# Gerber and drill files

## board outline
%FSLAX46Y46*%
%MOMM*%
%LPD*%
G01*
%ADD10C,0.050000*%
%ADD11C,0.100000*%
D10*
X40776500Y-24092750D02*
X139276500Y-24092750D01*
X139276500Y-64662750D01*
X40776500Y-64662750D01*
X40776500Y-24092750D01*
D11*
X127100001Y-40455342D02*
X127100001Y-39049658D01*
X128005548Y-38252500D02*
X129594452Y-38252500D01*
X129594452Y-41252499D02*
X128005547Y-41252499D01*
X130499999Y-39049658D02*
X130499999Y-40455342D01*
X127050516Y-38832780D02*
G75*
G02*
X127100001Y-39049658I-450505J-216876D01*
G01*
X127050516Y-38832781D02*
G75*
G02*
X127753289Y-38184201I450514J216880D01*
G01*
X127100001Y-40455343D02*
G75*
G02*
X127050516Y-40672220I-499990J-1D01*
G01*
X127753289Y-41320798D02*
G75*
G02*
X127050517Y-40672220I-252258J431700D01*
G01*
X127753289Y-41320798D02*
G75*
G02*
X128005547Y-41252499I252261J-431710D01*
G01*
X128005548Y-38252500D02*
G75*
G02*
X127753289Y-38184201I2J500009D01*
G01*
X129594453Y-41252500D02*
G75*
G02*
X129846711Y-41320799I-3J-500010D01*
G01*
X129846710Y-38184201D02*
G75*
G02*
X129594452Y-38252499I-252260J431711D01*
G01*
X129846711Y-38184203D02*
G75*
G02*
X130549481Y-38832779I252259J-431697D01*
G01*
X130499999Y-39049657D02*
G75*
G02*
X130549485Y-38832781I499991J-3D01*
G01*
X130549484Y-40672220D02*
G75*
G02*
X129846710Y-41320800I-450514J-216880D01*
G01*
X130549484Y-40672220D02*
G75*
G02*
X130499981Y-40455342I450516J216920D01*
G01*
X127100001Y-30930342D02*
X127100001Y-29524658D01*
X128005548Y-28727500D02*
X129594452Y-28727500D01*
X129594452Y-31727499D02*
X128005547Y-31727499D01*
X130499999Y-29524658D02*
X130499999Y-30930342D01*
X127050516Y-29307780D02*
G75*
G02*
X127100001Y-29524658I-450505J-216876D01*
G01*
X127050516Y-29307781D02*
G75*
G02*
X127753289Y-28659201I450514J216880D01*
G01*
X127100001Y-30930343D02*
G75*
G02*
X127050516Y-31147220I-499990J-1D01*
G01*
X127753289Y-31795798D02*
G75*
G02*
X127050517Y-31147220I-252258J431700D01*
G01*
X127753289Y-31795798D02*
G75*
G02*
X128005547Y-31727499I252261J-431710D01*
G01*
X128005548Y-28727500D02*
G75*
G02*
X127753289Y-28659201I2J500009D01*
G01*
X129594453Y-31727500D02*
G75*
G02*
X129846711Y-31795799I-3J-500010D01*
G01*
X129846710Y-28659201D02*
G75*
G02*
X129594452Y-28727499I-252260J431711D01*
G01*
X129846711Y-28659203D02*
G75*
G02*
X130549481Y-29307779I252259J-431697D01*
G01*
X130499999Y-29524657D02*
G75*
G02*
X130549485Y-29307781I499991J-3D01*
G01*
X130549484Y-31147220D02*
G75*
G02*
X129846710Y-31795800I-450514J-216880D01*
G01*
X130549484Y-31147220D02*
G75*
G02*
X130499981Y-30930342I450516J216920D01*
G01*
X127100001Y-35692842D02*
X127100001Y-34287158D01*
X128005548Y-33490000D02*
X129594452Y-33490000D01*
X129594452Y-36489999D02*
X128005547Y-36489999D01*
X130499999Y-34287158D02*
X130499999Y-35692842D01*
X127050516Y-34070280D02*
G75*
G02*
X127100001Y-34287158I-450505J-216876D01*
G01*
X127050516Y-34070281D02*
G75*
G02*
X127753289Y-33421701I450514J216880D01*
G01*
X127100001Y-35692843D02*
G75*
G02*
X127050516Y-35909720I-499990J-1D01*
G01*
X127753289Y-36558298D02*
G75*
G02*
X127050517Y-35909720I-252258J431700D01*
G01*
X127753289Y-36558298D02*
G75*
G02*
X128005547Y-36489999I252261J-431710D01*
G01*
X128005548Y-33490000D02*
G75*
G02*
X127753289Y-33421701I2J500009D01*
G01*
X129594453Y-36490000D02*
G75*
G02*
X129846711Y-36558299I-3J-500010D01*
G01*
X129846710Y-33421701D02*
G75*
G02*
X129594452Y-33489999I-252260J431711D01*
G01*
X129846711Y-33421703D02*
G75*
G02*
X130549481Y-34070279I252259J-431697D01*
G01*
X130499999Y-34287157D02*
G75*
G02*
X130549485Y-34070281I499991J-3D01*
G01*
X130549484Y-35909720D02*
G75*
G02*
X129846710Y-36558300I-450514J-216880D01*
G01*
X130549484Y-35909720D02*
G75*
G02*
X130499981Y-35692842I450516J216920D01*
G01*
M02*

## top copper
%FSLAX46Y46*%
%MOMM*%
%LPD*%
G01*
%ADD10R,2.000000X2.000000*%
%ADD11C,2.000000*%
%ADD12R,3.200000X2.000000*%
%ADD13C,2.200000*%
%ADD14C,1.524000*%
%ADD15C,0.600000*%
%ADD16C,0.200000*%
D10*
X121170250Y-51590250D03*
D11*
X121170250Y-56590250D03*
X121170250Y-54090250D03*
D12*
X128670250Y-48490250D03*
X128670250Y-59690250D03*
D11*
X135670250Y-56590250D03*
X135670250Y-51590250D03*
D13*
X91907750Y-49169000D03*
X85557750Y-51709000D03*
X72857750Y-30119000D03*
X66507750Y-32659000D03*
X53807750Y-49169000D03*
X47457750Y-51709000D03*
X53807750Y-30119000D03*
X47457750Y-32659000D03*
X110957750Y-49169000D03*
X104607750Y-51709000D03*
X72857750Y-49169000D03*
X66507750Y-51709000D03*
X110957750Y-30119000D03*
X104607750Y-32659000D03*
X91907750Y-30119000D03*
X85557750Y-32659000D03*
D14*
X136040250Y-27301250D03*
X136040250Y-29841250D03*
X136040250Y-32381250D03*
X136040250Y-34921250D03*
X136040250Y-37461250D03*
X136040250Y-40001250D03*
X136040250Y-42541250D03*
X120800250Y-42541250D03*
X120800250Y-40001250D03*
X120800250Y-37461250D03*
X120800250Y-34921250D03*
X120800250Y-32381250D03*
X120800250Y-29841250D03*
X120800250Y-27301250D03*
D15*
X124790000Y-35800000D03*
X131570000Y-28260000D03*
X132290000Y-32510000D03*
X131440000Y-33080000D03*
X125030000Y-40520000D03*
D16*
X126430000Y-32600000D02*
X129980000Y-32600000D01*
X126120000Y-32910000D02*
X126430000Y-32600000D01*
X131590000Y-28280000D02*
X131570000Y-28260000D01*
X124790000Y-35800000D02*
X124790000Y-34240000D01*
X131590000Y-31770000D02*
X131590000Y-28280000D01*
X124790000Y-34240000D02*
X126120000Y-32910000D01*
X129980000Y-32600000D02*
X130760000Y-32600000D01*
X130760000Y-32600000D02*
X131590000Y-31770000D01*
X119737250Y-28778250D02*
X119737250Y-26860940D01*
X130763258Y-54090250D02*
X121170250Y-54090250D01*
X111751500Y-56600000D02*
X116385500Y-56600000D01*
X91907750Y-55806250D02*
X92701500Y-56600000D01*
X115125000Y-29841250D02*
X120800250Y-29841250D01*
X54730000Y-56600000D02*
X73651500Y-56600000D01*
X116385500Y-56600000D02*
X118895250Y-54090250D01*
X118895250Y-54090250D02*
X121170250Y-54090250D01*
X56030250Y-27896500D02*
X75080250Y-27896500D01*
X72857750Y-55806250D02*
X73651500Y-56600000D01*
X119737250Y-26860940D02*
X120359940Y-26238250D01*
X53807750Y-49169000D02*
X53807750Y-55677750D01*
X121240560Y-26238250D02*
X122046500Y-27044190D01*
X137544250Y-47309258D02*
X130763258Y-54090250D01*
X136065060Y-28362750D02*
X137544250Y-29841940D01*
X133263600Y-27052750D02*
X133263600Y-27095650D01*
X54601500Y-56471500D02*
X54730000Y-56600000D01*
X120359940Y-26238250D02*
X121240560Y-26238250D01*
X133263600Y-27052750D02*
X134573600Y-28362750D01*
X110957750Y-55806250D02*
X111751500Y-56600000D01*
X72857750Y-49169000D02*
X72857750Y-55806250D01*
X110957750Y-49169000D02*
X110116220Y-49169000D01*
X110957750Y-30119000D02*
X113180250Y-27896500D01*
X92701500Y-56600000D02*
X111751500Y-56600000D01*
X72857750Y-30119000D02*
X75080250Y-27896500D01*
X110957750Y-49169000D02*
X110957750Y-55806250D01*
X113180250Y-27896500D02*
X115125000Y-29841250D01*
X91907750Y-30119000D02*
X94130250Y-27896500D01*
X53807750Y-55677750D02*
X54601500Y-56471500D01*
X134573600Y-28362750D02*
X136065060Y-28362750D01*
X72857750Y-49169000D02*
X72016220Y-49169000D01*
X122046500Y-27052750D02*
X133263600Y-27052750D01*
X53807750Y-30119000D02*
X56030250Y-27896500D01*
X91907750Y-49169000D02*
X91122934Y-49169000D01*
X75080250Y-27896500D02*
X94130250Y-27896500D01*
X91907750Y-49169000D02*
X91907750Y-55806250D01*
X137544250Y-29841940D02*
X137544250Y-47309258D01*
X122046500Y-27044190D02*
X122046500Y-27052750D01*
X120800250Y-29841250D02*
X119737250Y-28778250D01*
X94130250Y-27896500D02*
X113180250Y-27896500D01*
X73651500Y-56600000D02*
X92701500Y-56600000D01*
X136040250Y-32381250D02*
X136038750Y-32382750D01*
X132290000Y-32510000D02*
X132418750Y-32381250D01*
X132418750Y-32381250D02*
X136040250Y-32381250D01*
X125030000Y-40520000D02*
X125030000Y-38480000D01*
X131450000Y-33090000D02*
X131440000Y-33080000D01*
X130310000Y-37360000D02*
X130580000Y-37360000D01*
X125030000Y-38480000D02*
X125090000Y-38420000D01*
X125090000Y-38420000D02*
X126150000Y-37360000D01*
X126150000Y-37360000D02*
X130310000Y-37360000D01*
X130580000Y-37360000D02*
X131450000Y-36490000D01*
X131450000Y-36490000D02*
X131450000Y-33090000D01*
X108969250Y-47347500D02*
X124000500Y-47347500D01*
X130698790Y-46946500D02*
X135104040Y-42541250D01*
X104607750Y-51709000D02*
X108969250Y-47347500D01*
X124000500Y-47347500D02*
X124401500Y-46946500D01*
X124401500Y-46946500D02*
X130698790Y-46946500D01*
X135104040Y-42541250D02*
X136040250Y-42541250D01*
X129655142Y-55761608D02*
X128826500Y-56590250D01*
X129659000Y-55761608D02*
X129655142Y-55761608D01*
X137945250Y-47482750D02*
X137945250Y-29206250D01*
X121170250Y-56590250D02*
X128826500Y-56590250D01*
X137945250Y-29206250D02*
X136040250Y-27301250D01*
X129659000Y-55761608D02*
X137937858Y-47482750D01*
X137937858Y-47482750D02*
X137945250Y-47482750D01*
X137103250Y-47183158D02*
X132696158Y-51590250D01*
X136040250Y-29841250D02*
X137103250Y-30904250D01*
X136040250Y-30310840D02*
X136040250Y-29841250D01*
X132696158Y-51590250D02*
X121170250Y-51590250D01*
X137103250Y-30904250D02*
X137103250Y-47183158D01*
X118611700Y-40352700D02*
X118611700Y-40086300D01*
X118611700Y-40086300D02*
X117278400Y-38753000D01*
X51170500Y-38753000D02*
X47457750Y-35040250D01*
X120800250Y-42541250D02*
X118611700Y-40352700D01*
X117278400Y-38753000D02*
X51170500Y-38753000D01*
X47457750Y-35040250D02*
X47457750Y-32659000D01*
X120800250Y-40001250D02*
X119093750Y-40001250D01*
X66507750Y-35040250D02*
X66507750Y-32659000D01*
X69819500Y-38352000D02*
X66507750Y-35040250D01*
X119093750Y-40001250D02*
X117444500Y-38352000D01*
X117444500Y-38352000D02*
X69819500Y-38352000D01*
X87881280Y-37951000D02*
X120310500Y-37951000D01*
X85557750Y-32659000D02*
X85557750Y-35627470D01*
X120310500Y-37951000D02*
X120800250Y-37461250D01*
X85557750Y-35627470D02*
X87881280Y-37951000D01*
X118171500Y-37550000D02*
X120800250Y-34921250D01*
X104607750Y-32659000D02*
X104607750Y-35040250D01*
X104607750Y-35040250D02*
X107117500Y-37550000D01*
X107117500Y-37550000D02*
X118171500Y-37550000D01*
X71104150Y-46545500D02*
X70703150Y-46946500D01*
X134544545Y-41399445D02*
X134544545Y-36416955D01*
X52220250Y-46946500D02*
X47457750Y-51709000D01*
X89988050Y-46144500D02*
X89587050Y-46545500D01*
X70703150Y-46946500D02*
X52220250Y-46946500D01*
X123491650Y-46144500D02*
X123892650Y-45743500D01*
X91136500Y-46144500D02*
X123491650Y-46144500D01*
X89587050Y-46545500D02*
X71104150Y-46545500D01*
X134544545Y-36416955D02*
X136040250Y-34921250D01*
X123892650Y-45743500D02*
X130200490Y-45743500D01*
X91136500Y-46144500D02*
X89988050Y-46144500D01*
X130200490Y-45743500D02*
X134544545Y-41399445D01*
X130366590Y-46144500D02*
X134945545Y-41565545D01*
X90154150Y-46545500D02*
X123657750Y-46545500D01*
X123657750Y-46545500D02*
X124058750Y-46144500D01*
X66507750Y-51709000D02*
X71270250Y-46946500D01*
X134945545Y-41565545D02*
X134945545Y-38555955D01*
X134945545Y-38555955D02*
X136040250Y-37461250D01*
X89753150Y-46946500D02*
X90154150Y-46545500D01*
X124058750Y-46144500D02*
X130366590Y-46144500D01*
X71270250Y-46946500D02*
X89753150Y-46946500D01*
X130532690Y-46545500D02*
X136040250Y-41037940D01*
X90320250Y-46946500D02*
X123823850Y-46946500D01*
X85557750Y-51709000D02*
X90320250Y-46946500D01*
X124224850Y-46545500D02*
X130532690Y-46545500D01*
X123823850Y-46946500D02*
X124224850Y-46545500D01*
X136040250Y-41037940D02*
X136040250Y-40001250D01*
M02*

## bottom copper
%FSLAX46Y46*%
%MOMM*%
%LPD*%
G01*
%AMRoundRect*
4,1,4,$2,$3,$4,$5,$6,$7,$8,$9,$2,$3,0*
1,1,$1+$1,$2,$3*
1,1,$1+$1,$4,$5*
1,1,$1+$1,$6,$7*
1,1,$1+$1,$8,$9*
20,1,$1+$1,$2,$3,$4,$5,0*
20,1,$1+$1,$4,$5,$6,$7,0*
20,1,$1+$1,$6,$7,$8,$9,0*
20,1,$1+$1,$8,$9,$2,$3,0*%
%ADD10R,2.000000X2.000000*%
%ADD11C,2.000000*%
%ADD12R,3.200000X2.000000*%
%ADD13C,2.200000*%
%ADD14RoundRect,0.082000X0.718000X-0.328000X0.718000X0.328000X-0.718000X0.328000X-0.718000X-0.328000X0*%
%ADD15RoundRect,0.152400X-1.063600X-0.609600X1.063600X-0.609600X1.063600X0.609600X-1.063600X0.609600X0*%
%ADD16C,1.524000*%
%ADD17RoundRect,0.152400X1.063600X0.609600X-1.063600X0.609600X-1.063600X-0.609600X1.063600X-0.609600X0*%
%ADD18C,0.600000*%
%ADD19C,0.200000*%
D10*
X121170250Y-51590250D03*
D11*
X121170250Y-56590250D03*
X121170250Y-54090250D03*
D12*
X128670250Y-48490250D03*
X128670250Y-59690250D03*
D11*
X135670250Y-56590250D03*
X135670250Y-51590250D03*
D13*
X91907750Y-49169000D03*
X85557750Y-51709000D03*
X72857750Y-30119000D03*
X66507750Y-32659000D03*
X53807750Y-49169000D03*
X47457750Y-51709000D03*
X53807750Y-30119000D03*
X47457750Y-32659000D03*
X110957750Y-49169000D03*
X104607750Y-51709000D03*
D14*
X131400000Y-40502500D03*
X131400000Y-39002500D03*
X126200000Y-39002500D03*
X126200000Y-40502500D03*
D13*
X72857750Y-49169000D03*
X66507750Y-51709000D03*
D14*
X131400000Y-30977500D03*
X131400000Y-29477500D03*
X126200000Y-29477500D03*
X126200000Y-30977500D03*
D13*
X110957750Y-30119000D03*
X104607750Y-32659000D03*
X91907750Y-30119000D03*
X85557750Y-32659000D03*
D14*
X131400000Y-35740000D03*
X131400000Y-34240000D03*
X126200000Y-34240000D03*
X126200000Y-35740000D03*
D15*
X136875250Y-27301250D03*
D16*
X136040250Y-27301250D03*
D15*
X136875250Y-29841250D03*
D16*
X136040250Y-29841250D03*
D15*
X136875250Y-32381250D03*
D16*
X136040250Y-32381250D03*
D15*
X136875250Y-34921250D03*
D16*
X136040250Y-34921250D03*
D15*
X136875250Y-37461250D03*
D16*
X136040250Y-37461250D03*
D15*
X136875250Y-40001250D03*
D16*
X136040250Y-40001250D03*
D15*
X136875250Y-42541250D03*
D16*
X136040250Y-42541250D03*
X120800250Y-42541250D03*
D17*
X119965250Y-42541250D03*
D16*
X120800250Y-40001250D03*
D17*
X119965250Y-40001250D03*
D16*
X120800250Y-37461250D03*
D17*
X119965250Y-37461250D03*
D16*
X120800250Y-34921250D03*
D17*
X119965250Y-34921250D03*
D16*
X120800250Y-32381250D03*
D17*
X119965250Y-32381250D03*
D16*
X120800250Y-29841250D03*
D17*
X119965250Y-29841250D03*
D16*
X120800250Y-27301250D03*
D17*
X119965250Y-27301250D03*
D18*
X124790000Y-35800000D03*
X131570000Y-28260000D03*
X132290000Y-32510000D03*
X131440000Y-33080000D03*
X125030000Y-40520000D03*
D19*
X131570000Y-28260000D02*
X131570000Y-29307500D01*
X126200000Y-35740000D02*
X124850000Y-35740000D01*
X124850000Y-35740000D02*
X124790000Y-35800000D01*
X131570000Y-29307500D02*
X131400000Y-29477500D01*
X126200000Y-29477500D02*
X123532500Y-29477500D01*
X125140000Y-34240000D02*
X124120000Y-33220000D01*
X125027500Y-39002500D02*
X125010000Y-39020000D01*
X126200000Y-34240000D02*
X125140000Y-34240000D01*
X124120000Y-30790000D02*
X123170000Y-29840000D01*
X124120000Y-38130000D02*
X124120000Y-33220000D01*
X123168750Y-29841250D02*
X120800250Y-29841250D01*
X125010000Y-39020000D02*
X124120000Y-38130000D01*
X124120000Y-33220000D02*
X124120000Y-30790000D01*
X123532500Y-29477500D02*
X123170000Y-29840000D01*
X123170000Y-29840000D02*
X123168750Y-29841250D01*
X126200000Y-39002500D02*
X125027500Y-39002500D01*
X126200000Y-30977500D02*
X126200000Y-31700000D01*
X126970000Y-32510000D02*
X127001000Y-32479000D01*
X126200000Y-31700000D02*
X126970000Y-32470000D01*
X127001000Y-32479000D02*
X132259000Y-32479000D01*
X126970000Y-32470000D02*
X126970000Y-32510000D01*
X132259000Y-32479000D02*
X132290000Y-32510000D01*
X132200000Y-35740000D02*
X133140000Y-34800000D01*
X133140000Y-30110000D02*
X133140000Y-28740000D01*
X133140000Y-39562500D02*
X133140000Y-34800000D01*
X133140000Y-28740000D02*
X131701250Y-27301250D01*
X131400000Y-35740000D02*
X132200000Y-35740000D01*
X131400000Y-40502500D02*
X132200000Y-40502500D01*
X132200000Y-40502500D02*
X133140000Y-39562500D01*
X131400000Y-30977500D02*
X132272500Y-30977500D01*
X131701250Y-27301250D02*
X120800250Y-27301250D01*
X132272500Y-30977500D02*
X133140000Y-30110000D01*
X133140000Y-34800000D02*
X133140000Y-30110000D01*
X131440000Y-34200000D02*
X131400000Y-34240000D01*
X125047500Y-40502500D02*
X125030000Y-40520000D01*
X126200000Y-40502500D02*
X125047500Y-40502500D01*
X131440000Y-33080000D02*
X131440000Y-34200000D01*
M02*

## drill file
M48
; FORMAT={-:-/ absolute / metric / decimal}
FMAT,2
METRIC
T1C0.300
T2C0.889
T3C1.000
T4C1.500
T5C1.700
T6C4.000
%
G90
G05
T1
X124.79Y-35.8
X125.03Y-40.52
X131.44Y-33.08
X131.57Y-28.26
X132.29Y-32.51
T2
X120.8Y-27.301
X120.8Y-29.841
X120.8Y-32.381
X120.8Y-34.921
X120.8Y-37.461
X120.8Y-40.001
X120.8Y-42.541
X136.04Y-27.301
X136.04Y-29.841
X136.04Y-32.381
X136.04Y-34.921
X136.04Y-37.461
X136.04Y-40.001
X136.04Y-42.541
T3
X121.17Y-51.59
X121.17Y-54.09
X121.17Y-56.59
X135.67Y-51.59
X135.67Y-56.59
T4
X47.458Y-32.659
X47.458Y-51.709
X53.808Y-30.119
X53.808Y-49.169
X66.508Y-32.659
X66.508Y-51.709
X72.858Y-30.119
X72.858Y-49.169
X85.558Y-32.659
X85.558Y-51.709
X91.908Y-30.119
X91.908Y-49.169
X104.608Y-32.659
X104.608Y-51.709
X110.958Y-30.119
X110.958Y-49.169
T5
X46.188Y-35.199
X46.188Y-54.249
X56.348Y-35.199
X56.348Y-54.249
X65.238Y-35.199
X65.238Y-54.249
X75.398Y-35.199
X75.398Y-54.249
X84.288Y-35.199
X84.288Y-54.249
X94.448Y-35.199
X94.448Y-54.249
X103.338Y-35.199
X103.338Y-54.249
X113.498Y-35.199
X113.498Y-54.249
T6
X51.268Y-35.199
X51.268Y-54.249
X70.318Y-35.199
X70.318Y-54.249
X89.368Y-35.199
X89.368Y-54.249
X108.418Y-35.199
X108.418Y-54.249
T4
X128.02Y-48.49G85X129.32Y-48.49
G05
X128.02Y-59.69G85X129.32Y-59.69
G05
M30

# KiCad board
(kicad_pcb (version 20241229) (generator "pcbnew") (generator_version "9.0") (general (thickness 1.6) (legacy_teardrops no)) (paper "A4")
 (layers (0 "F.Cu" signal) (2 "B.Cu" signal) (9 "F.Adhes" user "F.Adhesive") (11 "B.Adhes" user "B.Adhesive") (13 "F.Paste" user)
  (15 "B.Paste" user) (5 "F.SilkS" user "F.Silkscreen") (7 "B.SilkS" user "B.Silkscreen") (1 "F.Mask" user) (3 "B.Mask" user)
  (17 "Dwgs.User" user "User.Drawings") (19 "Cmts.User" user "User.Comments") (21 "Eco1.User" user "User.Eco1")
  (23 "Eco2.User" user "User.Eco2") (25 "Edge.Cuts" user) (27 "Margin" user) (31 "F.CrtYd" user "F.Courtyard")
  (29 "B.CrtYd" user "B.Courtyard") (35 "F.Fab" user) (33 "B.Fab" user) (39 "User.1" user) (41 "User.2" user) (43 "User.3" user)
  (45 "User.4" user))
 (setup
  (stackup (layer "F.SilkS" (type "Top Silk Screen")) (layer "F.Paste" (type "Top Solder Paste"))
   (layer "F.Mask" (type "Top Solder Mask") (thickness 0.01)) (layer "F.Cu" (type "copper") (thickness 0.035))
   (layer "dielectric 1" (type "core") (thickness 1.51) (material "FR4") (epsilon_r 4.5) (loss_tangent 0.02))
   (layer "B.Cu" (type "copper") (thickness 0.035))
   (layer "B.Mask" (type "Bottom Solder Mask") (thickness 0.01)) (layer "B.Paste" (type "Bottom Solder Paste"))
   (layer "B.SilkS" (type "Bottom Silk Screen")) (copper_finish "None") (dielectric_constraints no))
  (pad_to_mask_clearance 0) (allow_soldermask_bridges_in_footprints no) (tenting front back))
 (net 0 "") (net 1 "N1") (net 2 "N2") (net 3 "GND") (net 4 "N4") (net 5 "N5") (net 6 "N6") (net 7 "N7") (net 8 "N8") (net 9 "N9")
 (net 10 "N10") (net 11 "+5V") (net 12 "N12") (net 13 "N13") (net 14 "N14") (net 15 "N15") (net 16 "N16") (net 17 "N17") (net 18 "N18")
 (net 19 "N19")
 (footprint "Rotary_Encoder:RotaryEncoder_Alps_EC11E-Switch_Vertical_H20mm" (layer "F.Cu") (at 121.17025 51.59025)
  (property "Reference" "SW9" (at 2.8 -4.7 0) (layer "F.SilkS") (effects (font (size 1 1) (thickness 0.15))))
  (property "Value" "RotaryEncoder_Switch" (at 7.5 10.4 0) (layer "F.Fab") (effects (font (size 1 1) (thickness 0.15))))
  (pad "A" thru_hole rect (at 0 0) (size 2 2) (drill 1) (layers "*.Cu" "*.Mask") (remove_unused_layers no) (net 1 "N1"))
  (pad "B" thru_hole circle (at 0 5) (size 2 2) (drill 1) (layers "*.Cu" "*.Mask") (remove_unused_layers no) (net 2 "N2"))
  (pad "C" thru_hole circle (at 0 2.5) (size 2 2) (drill 1) (layers "*.Cu" "*.Mask") (remove_unused_layers no) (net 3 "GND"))
  (pad "MP" thru_hole rect (at 7.5 -3.1) (size 3.2 2) (drill oval 2.8 1.5) (layers "*.Cu" "*.Mask") (remove_unused_layers no))
  (pad "MP" thru_hole rect (at 7.5 8.1) (size 3.2 2) (drill oval 2.8 1.5) (layers "*.Cu" "*.Mask") (remove_unused_layers no))
  (pad "S1" thru_hole circle (at 14.5 5) (size 2 2) (drill 1) (layers "*.Cu" "*.Mask") (remove_unused_layers no) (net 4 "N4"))
  (pad "S2" thru_hole circle (at 14.5 0) (size 2 2) (drill 1) (layers "*.Cu" "*.Mask") (remove_unused_layers no) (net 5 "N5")))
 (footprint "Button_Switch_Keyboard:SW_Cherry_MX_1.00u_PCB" (layer "F.Cu") (at 91.90775 49.169)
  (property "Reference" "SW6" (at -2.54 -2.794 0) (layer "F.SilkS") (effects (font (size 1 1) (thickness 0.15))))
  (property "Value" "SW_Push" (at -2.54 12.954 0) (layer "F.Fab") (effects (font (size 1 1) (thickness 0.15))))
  (pad "" np_thru_hole circle (at -7.62 5.08) (size 1.7 1.7) (drill 1.7) (layers "*.Cu" "*.Mask"))
  (pad "" np_thru_hole circle (at -2.54 5.08) (size 4 4) (drill 4) (layers "*.Cu" "*.Mask"))
  (pad "" np_thru_hole circle (at 2.54 5.08) (size 1.7 1.7) (drill 1.7) (layers "*.Cu" "*.Mask"))
  (pad "1" thru_hole circle (at 0 0) (size 2.2 2.2) (drill 1.5) (layers "*.Cu" "*.Mask") (remove_unused_layers no) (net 3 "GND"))
  (pad "2" thru_hole circle (at -6.35 2.54) (size 2.2 2.2) (drill 1.5) (layers "*.Cu" "*.Mask") (remove_unused_layers no) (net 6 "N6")))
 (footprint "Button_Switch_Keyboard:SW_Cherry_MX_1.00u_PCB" (layer "F.Cu") (at 72.85775 30.119)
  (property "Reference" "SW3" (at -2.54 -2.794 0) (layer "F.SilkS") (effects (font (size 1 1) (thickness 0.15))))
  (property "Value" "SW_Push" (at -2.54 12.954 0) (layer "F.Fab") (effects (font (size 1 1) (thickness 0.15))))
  (pad "" np_thru_hole circle (at -7.62 5.08) (size 1.7 1.7) (drill 1.7) (layers "*.Cu" "*.Mask"))
  (pad "" np_thru_hole circle (at -2.54 5.08) (size 4 4) (drill 4) (layers "*.Cu" "*.Mask"))
  (pad "" np_thru_hole circle (at 2.54 5.08) (size 1.7 1.7) (drill 1.7) (layers "*.Cu" "*.Mask"))
  (pad "1" thru_hole circle (at 0 0) (size 2.2 2.2) (drill 1.5) (layers "*.Cu" "*.Mask") (remove_unused_layers no) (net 3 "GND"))
  (pad "2" thru_hole circle (at -6.35 2.54) (size 2.2 2.2) (drill 1.5) (layers "*.Cu" "*.Mask") (remove_unused_layers no) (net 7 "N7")))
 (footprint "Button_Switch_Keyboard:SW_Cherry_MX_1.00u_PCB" (layer "F.Cu") (at 53.80775 49.169)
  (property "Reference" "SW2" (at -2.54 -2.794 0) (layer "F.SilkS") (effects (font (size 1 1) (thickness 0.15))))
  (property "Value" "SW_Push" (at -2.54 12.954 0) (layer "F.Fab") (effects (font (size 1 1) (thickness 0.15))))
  (pad "" np_thru_hole circle (at -7.62 5.08) (size 1.7 1.7) (drill 1.7) (layers "*.Cu" "*.Mask"))
  (pad "" np_thru_hole circle (at -2.54 5.08) (size 4 4) (drill 4) (layers "*.Cu" "*.Mask"))
  (pad "" np_thru_hole circle (at 2.54 5.08) (size 1.7 1.7) (drill 1.7) (layers "*.Cu" "*.Mask"))
  (pad "1" thru_hole circle (at 0 0) (size 2.2 2.2) (drill 1.5) (layers "*.Cu" "*.Mask") (remove_unused_layers no) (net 3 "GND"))
  (pad "2" thru_hole circle (at -6.35 2.54) (size 2.2 2.2) (drill 1.5) (layers "*.Cu" "*.Mask") (remove_unused_layers no) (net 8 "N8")))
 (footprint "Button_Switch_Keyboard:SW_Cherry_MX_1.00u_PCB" (layer "F.Cu") (at 53.80775 30.119)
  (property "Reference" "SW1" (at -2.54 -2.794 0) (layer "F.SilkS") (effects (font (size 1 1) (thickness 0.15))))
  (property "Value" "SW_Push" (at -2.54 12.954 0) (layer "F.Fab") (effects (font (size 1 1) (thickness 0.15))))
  (pad "" np_thru_hole circle (at -7.62 5.08) (size 1.7 1.7) (drill 1.7) (layers "*.Cu" "*.Mask"))
  (pad "" np_thru_hole circle (at -2.54 5.08) (size 4 4) (drill 4) (layers "*.Cu" "*.Mask"))
  (pad "" np_thru_hole circle (at 2.54 5.08) (size 1.7 1.7) (drill 1.7) (layers "*.Cu" "*.Mask"))
  (pad "1" thru_hole circle (at 0 0) (size 2.2 2.2) (drill 1.5) (layers "*.Cu" "*.Mask") (remove_unused_layers no) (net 3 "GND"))
  (pad "2" thru_hole circle (at -6.35 2.54) (size 2.2 2.2) (drill 1.5) (layers "*.Cu" "*.Mask") (remove_unused_layers no) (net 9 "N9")))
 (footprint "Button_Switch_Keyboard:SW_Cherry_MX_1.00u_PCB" (layer "F.Cu") (at 110.95775 49.169)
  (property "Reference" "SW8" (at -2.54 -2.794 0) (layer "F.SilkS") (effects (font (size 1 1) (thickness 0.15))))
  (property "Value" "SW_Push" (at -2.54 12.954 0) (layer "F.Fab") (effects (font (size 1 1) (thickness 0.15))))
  (pad "" np_thru_hole circle (at -7.62 5.08) (size 1.7 1.7) (drill 1.7) (layers "*.Cu" "*.Mask"))
  (pad "" np_thru_hole circle (at -2.54 5.08) (size 4 4) (drill 4) (layers "*.Cu" "*.Mask"))
  (pad "" np_thru_hole circle (at 2.54 5.08) (size 1.7 1.7) (drill 1.7) (layers "*.Cu" "*.Mask"))
  (pad "1" thru_hole circle (at 0 0) (size 2.2 2.2) (drill 1.5) (layers "*.Cu" "*.Mask") (remove_unused_layers no) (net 3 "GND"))
  (pad "2" thru_hole circle (at -6.35 2.54) (size 2.2 2.2) (drill 1.5) (layers "*.Cu" "*.Mask") (remove_unused_layers no) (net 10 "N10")))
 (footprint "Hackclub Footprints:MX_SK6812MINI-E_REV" (layer "F.Cu") (at 128.8 34.6725)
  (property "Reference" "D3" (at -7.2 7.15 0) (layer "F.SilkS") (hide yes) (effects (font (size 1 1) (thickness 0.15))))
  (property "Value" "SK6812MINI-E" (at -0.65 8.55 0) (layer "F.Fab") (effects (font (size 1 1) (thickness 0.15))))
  (fp_line (start -1.699999 5.782842) (end -1.699999 4.377158) (stroke (width 0.1) (type solid)) (layer "Edge.Cuts"))
  (fp_line (start -0.794452 3.58) (end 0.794452 3.58) (stroke (width 0.1) (type solid)) (layer "Edge.Cuts"))
  (fp_line (start 0.794452 6.579999) (end -0.794453 6.579999) (stroke (width 0.1) (type solid)) (layer "Edge.Cuts"))
  (fp_line (start 1.699999 4.377158) (end 1.699999 5.782842) (stroke (width 0.1) (type solid)) (layer "Edge.Cuts"))
  (fp_arc (start -1.749484 4.16028) (mid -1.712527 4.265932) (end -1.699999 4.377158) (stroke (width 0.1) (type solid)) (layer "Edge.Cuts"))
  (fp_arc (start -1.749484 4.160281) (mid -1.638072 3.575965) (end -1.046711 3.511701) (stroke (width 0.1) (type solid)) (layer "Edge.Cuts"))
  (fp_arc (start -1.699999 5.782843) (mid -1.712527 5.894068) (end -1.749484 5.99972) (stroke (width 0.1) (type solid)) (layer "Edge.Cuts"))
  (fp_arc (start -1.046711 6.648298) (mid -1.638071 6.584034) (end -1.749484 5.99972) (stroke (width 0.1) (type solid)) (layer "Edge.Cuts"))
  (fp_arc (start -1.046711 6.648298) (mid -0.925123 6.597376) (end -0.794453 6.579999) (stroke (width 0.1) (type solid)) (layer "Edge.Cuts"))
  (fp_arc (start -0.794452 3.58) (mid -0.925123 3.562623) (end -1.046711 3.511701) (stroke (width 0.1) (type solid)) (layer "Edge.Cuts"))
  (fp_arc (start 0.794453 6.58) (mid 0.925123 6.597377) (end 1.046711 6.648299) (stroke (width 0.1) (type solid)) (layer "Edge.Cuts"))
  (fp_arc (start 1.04671 3.511701) (mid 0.925122 3.562623) (end 0.794452 3.58) (stroke (width 0.1) (type solid)) (layer "Edge.Cuts"))
  (fp_arc (start 1.046711 3.511703) (mid 1.63807 3.575966) (end 1.749484 4.16028) (stroke (width 0.1) (type solid)) (layer "Edge.Cuts"))
  (fp_arc (start 1.699999 4.377157) (mid 1.712527 4.265932) (end 1.749484 4.16028) (stroke (width 0.1) (type solid)) (layer "Edge.Cuts"))
  (fp_arc (start 1.749484 5.99972) (mid 1.638071 6.584035) (end 1.046711 6.648299) (stroke (width 0.1) (type solid)) (layer "Edge.Cuts"))
  (fp_arc (start 1.749484 5.99972) (mid 1.712527 5.894068) (end 1.699999 5.782842) (stroke (width 0.1) (type solid)) (layer "Edge.Cuts"))
  (pad "1" smd roundrect (at 2.6 5.83 90) (size 0.82 1.6) (layers "B.Cu" "B.Mask" "B.Paste") (roundrect_rratio 0.1) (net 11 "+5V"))
  (pad "2" smd roundrect (at 2.6 4.33 90) (size 0.82 1.6) (layers "B.Cu" "B.Mask" "B.Paste") (roundrect_rratio 0.1) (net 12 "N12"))
  (pad "3" smd roundrect (at -2.6 4.33 90) (size 0.82 1.6) (layers "B.Cu" "B.Mask" "B.Paste") (roundrect_rratio 0.1) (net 3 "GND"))
  (pad "4" smd roundrect (at -2.6 5.83 90) (size 0.82 1.6) (layers "B.Cu" "B.Mask" "B.Paste") (roundrect_rratio 0.1) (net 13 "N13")))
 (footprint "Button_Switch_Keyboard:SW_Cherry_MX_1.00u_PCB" (layer "F.Cu") (at 72.85775 49.169)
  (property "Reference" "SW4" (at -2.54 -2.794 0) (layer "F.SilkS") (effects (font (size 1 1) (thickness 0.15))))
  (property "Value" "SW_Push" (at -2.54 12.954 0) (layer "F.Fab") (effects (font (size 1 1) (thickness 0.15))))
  (pad "" np_thru_hole circle (at -7.62 5.08) (size 1.7 1.7) (drill 1.7) (layers "*.Cu" "*.Mask"))
  (pad "" np_thru_hole circle (at -2.54 5.08) (size 4 4) (drill 4) (layers "*.Cu" "*.Mask"))
  (pad "" np_thru_hole circle (at 2.54 5.08) (size 1.7 1.7) (drill 1.7) (layers "*.Cu" "*.Mask"))
  (pad "1" thru_hole circle (at 0 0) (size 2.2 2.2) (drill 1.5) (layers "*.Cu" "*.Mask") (remove_unused_layers no) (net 3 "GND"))
  (pad "2" thru_hole circle (at -6.35 2.54) (size 2.2 2.2) (drill 1.5) (layers "*.Cu" "*.Mask") (remove_unused_layers no) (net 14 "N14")))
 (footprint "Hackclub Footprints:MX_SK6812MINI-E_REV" (layer "F.Cu") (at 128.8 25.1475)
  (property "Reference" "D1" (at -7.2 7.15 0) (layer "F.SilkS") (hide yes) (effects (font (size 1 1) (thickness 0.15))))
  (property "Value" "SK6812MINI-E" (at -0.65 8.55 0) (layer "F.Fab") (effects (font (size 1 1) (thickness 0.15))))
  (fp_line (start -1.699999 5.782842) (end -1.699999 4.377158) (stroke (width 0.1) (type solid)) (layer "Edge.Cuts"))
  (fp_line (start -0.794452 3.58) (end 0.794452 3.58) (stroke (width 0.1) (type solid)) (layer "Edge.Cuts"))
  (fp_line (start 0.794452 6.579999) (end -0.794453 6.579999) (stroke (width 0.1) (type solid)) (layer "Edge.Cuts"))
  (fp_line (start 1.699999 4.377158) (end 1.699999 5.782842) (stroke (width 0.1) (type solid)) (layer "Edge.Cuts"))
  (fp_arc (start -1.749484 4.16028) (mid -1.712527 4.265932) (end -1.699999 4.377158) (stroke (width 0.1) (type solid)) (layer "Edge.Cuts"))
  (fp_arc (start -1.749484 4.160281) (mid -1.638072 3.575965) (end -1.046711 3.511701) (stroke (width 0.1) (type solid)) (layer "Edge.Cuts"))
  (fp_arc (start -1.699999 5.782843) (mid -1.712527 5.894068) (end -1.749484 5.99972) (stroke (width 0.1) (type solid)) (layer "Edge.Cuts"))
  (fp_arc (start -1.046711 6.648298) (mid -1.638071 6.584034) (end -1.749484 5.99972) (stroke (width 0.1) (type solid)) (layer "Edge.Cuts"))
  (fp_arc (start -1.046711 6.648298) (mid -0.925123 6.597376) (end -0.794453 6.579999) (stroke (width 0.1) (type solid)) (layer "Edge.Cuts"))
  (fp_arc (start -0.794452 3.58) (mid -0.925123 3.562623) (end -1.046711 3.511701) (stroke (width 0.1) (type solid)) (layer "Edge.Cuts"))
  (fp_arc (start 0.794453 6.58) (mid 0.925123 6.597377) (end 1.046711 6.648299) (stroke (width 0.1) (type solid)) (layer "Edge.Cuts"))
  (fp_arc (start 1.04671 3.511701) (mid 0.925122 3.562623) (end 0.794452 3.58) (stroke (width 0.1) (type solid)) (layer "Edge.Cuts"))
  (fp_arc (start 1.046711 3.511703) (mid 1.63807 3.575966) (end 1.749484 4.16028) (stroke (width 0.1) (type solid)) (layer "Edge.Cuts"))
  (fp_arc (start 1.699999 4.377157) (mid 1.712527 4.265932) (end 1.749484 4.16028) (stroke (width 0.1) (type solid)) (layer "Edge.Cuts"))
  (fp_arc (start 1.749484 5.99972) (mid 1.638071 6.584035) (end 1.046711 6.648299) (stroke (width 0.1) (type solid)) (layer "Edge.Cuts"))
  (fp_arc (start 1.749484 5.99972) (mid 1.712527 5.894068) (end 1.699999 5.782842) (stroke (width 0.1) (type solid)) (layer "Edge.Cuts"))
  (pad "1" smd roundrect (at 2.6 5.83 90) (size 0.82 1.6) (layers "B.Cu" "B.Mask" "B.Paste") (roundrect_rratio 0.1) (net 11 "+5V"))
  (pad "2" smd roundrect (at 2.6 4.33 90) (size 0.82 1.6) (layers "B.Cu" "B.Mask" "B.Paste") (roundrect_rratio 0.1) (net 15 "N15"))
  (pad "3" smd roundrect (at -2.6 4.33 90) (size 0.82 1.6) (layers "B.Cu" "B.Mask" "B.Paste") (roundrect_rratio 0.1) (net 3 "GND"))
  (pad "4" smd roundrect (at -2.6 5.83 90) (size 0.82 1.6) (layers "B.Cu" "B.Mask" "B.Paste") (roundrect_rratio 0.1) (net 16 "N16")))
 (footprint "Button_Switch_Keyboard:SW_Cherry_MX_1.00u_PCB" (layer "F.Cu") (at 110.95775 30.119)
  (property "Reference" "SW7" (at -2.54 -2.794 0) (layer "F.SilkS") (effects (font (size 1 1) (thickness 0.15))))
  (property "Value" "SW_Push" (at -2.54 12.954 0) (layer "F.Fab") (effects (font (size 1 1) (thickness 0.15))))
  (pad "" np_thru_hole circle (at -7.62 5.08) (size 1.7 1.7) (drill 1.7) (layers "*.Cu" "*.Mask"))
  (pad "" np_thru_hole circle (at -2.54 5.08) (size 4 4) (drill 4) (layers "*.Cu" "*.Mask"))
  (pad "" np_thru_hole circle (at 2.54 5.08) (size 1.7 1.7) (drill 1.7) (layers "*.Cu" "*.Mask"))
  (pad "1" thru_hole circle (at 0 0) (size 2.2 2.2) (drill 1.5) (layers "*.Cu" "*.Mask") (remove_unused_layers no) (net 3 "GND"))
  (pad "2" thru_hole circle (at -6.35 2.54) (size 2.2 2.2) (drill 1.5) (layers "*.Cu" "*.Mask") (remove_unused_layers no) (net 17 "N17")))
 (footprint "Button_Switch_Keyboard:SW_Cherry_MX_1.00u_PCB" (layer "F.Cu") (at 91.90775 30.119)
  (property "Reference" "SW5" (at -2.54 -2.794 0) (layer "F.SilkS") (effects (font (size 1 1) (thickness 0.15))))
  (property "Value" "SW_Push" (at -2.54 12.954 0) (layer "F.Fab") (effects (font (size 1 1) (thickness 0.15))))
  (pad "" np_thru_hole circle (at -7.62 5.08) (size 1.7 1.7) (drill 1.7) (layers "*.Cu" "*.Mask"))
  (pad "" np_thru_hole circle (at -2.54 5.08) (size 4 4) (drill 4) (layers "*.Cu" "*.Mask"))
  (pad "" np_thru_hole circle (at 2.54 5.08) (size 1.7 1.7) (drill 1.7) (layers "*.Cu" "*.Mask"))
  (pad "1" thru_hole circle (at 0 0) (size 2.2 2.2) (drill 1.5) (layers "*.Cu" "*.Mask") (remove_unused_layers no) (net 3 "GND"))
  (pad "2" thru_hole circle (at -6.35 2.54) (size 2.2 2.2) (drill 1.5) (layers "*.Cu" "*.Mask") (remove_unused_layers no) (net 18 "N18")))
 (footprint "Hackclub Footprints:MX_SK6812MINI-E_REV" (layer "F.Cu") (at 128.8 29.91)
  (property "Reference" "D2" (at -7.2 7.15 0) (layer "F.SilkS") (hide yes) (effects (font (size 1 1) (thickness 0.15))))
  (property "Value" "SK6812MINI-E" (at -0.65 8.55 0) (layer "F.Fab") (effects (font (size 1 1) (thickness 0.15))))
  (fp_line (start -1.699999 5.782842) (end -1.699999 4.377158) (stroke (width 0.1) (type solid)) (layer "Edge.Cuts"))
  (fp_line (start -0.794452 3.58) (end 0.794452 3.58) (stroke (width 0.1) (type solid)) (layer "Edge.Cuts"))
  (fp_line (start 0.794452 6.579999) (end -0.794453 6.579999) (stroke (width 0.1) (type solid)) (layer "Edge.Cuts"))
  (fp_line (start 1.699999 4.377158) (end 1.699999 5.782842) (stroke (width 0.1) (type solid)) (layer "Edge.Cuts"))
  (fp_arc (start -1.749484 4.16028) (mid -1.712527 4.265932) (end -1.699999 4.377158) (stroke (width 0.1) (type solid)) (layer "Edge.Cuts"))
  (fp_arc (start -1.749484 4.160281) (mid -1.638072 3.575965) (end -1.046711 3.511701) (stroke (width 0.1) (type solid)) (layer "Edge.Cuts"))
  (fp_arc (start -1.699999 5.782843) (mid -1.712527 5.894068) (end -1.749484 5.99972) (stroke (width 0.1) (type solid)) (layer "Edge.Cuts"))
  (fp_arc (start -1.046711 6.648298) (mid -1.638071 6.584034) (end -1.749484 5.99972) (stroke (width 0.1) (type solid)) (layer "Edge.Cuts"))
  (fp_arc (start -1.046711 6.648298) (mid -0.925123 6.597376) (end -0.794453 6.579999) (stroke (width 0.1) (type solid)) (layer "Edge.Cuts"))
  (fp_arc (start -0.794452 3.58) (mid -0.925123 3.562623) (end -1.046711 3.511701) (stroke (width 0.1) (type solid)) (layer "Edge.Cuts"))
  (fp_arc (start 0.794453 6.58) (mid 0.925123 6.597377) (end 1.046711 6.648299) (stroke (width 0.1) (type solid)) (layer "Edge.Cuts"))
  (fp_arc (start 1.04671 3.511701) (mid 0.925122 3.562623) (end 0.794452 3.58) (stroke (width 0.1) (type solid)) (layer "Edge.Cuts"))
  (fp_arc (start 1.046711 3.511703) (mid 1.63807 3.575966) (end 1.749484 4.16028) (stroke (width 0.1) (type solid)) (layer "Edge.Cuts"))
  (fp_arc (start 1.699999 4.377157) (mid 1.712527 4.265932) (end 1.749484 4.16028) (stroke (width 0.1) (type solid)) (layer "Edge.Cuts"))
  (fp_arc (start 1.749484 5.99972) (mid 1.638071 6.584035) (end 1.046711 6.648299) (stroke (width 0.1) (type solid)) (layer "Edge.Cuts"))
  (fp_arc (start 1.749484 5.99972) (mid 1.712527 5.894068) (end 1.699999 5.782842) (stroke (width 0.1) (type solid)) (layer "Edge.Cuts"))
  (pad "1" smd roundrect (at 2.6 5.83 90) (size 0.82 1.6) (layers "B.Cu" "B.Mask" "B.Paste") (roundrect_rratio 0.1) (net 11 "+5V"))
  (pad "2" smd roundrect (at 2.6 4.33 90) (size 0.82 1.6) (layers "B.Cu" "B.Mask" "B.Paste") (roundrect_rratio 0.1) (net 13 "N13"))
  (pad "3" smd roundrect (at -2.6 4.33 90) (size 0.82 1.6) (layers "B.Cu" "B.Mask" "B.Paste") (roundrect_rratio 0.1) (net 3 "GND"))
  (pad "4" smd roundrect (at -2.6 5.83 90) (size 0.82 1.6) (layers "B.Cu" "B.Mask" "B.Paste") (roundrect_rratio 0.1) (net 15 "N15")))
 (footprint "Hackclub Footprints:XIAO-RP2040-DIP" (layer "B.Cu") (at 128.42025 34.92125 180)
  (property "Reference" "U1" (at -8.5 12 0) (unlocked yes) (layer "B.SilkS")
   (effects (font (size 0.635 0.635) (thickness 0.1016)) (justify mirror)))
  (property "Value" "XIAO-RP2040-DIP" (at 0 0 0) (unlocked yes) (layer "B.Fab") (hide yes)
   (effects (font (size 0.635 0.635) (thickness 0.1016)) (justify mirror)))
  (pad "1" smd roundrect (at -8.455 7.62) (size 2.432 1.524) (layers "B.Cu" "B.Mask") (roundrect_rratio 0.1) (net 2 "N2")
   (thermal_bridge_angle 45))
  (pad "1" thru_hole circle (at -7.62 7.62) (size 1.524 1.524) (drill 0.889) (layers "*.Cu" "*.Mask") (remove_unused_layers no) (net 2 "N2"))
  (pad "2" smd roundrect (at -8.455 5.08) (size 2.432 1.524) (layers "B.Cu" "B.Mask") (roundrect_rratio 0.1) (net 1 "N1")
   (thermal_bridge_angle 45))
  (pad "2" thru_hole circle (at -7.62 5.08) (size 1.524 1.524) (drill 0.889) (layers "*.Cu" "*.Mask") (remove_unused_layers no) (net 1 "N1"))
  (pad "3" smd roundrect (at -8.455 2.54) (size 2.432 1.524) (layers "B.Cu" "B.Mask") (roundrect_rratio 0.1) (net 16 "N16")
   (thermal_bridge_angle 45))
  (pad "3" thru_hole circle (at -7.62 2.54) (size 1.524 1.524) (drill 0.889) (layers "*.Cu" "*.Mask") (remove_unused_layers no)
   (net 16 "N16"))
  (pad "4" smd roundrect (at -8.455 0) (size 2.432 1.524) (layers "B.Cu" "B.Mask") (roundrect_rratio 0.1) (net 8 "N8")
   (thermal_bridge_angle 45))
  (pad "4" thru_hole circle (at -7.62 0) (size 1.524 1.524) (drill 0.889) (layers "*.Cu" "*.Mask") (remove_unused_layers no) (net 8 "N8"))
  (pad "5" smd roundrect (at -8.455 -2.54) (size 2.432 1.524) (layers "B.Cu" "B.Mask") (roundrect_rratio 0.1) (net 14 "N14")
   (thermal_bridge_angle 45))
  (pad "5" thru_hole circle (at -7.62 -2.54) (size 1.524 1.524) (drill 0.889) (layers "*.Cu" "*.Mask") (remove_unused_layers no)
   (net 14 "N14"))
  (pad "6" smd roundrect (at -8.455 -5.08) (size 2.432 1.524) (layers "B.Cu" "B.Mask") (roundrect_rratio 0.1) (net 6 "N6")
   (thermal_bridge_angle 45))
  (pad "6" thru_hole circle (at -7.62 -5.08) (size 1.524 1.524) (drill 0.889) (layers "*.Cu" "*.Mask") (remove_unused_layers no)
   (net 6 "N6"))
  (pad "7" smd roundrect (at -8.455 -7.62) (size 2.432 1.524) (layers "B.Cu" "B.Mask") (roundrect_rratio 0.1) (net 10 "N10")
   (thermal_bridge_angle 45))
  (pad "7" thru_hole circle (at -7.62 -7.62) (size 1.524 1.524) (drill 0.889) (layers "*.Cu" "*.Mask") (remove_unused_layers no)
   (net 10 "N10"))
  (pad "8" thru_hole circle (at 7.62 -7.62 180) (size 1.524 1.524) (drill 0.889) (layers "*.Cu" "*.Mask") (remove_unused_layers no)
   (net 9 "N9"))
  (pad "8" smd roundrect (at 8.455 -7.62 180) (size 2.432 1.524) (layers "B.Cu" "B.Mask") (roundrect_rratio 0.1) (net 9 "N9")
   (thermal_bridge_angle 45))
  (pad "9" thru_hole circle (at 7.62 -5.08 180) (size 1.524 1.524) (drill 0.889) (layers "*.Cu" "*.Mask") (remove_unused_layers no)
   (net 7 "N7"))
  (pad "9" smd roundrect (at 8.455 -5.08 180) (size 2.432 1.524) (layers "B.Cu" "B.Mask") (roundrect_rratio 0.1) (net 7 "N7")
   (thermal_bridge_angle 45))
  (pad "10" thru_hole circle (at 7.62 -2.54 180) (size 1.524 1.524) (drill 0.889) (layers "*.Cu" "*.Mask") (remove_unused_layers no)
   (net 18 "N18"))
  (pad "10" smd roundrect (at 8.455 -2.54 180) (size 2.432 1.524) (layers "B.Cu" "B.Mask") (roundrect_rratio 0.1) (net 18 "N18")
   (thermal_bridge_angle 45))
  (pad "11" thru_hole circle (at 7.62 0 180) (size 1.524 1.524) (drill 0.889) (layers "*.Cu" "*.Mask") (remove_unused_layers no)
   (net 17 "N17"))
  (pad "11" smd roundrect (at 8.455 0 180) (size 2.432 1.524) (layers "B.Cu" "B.Mask") (roundrect_rratio 0.1) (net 17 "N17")
   (thermal_bridge_angle 45))
  (pad "12" thru_hole circle (at 7.62 2.54 180) (size 1.524 1.524) (drill 0.889) (layers "*.Cu" "*.Mask") (remove_unused_layers no)
   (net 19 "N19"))
  (pad "12" smd roundrect (at 8.455 2.54 180) (size 2.432 1.524) (layers "B.Cu" "B.Mask") (roundrect_rratio 0.1) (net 19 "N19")
   (thermal_bridge_angle 45))
  (pad "13" thru_hole circle (at 7.62 5.08 180) (size 1.524 1.524) (drill 0.889) (layers "*.Cu" "*.Mask") (remove_unused_layers no)
   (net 3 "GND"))
  (pad "13" smd roundrect (at 8.455 5.08 180) (size 2.432 1.524) (layers "B.Cu" "B.Mask") (roundrect_rratio 0.1) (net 3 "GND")
   (thermal_bridge_angle 45))
  (pad "14" thru_hole circle (at 7.62 7.62 180) (size 1.524 1.524) (drill 0.889) (layers "*.Cu" "*.Mask") (remove_unused_layers no)
   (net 11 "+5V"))
  (pad "14" smd roundrect (at 8.455 7.62 180) (size 2.432 1.524) (layers "B.Cu" "B.Mask") (roundrect_rratio 0.1) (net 11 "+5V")
   (thermal_bridge_angle 45)))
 (gr_rect (start 40.7765 24.09275) (end 139.2765 64.66275) (stroke (width 0.05) (type default)) (fill no) (layer "Edge.Cuts"))
 (segment (start 126.43 32.6) (end 129.98 32.6) (width 0.2) (layer "F.Cu") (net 15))
 (segment (start 126.12 32.91) (end 126.43 32.6) (width 0.2) (layer "F.Cu") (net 15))
 (segment (start 131.59 28.28) (end 131.57 28.26) (width 0.2) (layer "F.Cu") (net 15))
 (segment (start 124.79 35.8) (end 124.79 34.24) (width 0.2) (layer "F.Cu") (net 15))
 (segment (start 131.59 31.77) (end 131.59 28.28) (width 0.2) (layer "F.Cu") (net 15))
 (segment (start 124.79 34.24) (end 126.12 32.91) (width 0.2) (layer "F.Cu") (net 15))
 (segment (start 129.98 32.6) (end 130.76 32.6) (width 0.2) (layer "F.Cu") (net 15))
 (segment (start 130.76 32.6) (end 131.59 31.77) (width 0.2) (layer "F.Cu") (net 15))
 (via (at 124.79 35.8) (size 0.6) (drill 0.3) (layers "F.Cu" "B.Cu") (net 15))
 (via (at 131.57 28.26) (size 0.6) (drill 0.3) (layers "F.Cu" "B.Cu") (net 15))
 (segment (start 131.57 28.26) (end 131.57 29.3075) (width 0.2) (layer "B.Cu") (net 15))
 (segment (start 126.2 35.74) (end 124.85 35.74) (width 0.2) (layer "B.Cu") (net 15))
 (segment (start 124.85 35.74) (end 124.79 35.8) (width 0.2) (layer "B.Cu") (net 15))
 (segment (start 131.57 29.3075) (end 131.4 29.4775) (width 0.2) (layer "B.Cu") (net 15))
 (segment (start 119.73725 28.77825) (end 119.73725 26.86094) (width 0.2) (layer "F.Cu") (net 3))
 (segment (start 130.763258 54.09025) (end 121.17025 54.09025) (width 0.2) (layer "F.Cu") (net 3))
 (segment (start 111.7515 56.6) (end 116.3855 56.6) (width 0.2) (layer "F.Cu") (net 3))
 (segment (start 91.90775 55.80625) (end 92.7015 56.6) (width 0.2) (layer "F.Cu") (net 3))
 (segment (start 115.125 29.84125) (end 120.80025 29.84125) (width 0.2) (layer "F.Cu") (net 3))
 (segment (start 54.73 56.6) (end 73.6515 56.6) (width 0.2) (layer "F.Cu") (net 3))
 (segment (start 116.3855 56.6) (end 118.89525 54.09025) (width 0.2) (layer "F.Cu") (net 3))
 (segment (start 118.89525 54.09025) (end 121.17025 54.09025) (width 0.2) (layer "F.Cu") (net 3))
 (segment (start 56.03025 27.8965) (end 75.08025 27.8965) (width 0.2) (layer "F.Cu") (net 3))
 (segment (start 72.85775 55.80625) (end 73.6515 56.6) (width 0.2) (layer "F.Cu") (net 3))
 (segment (start 119.73725 26.86094) (end 120.35994 26.23825) (width 0.2) (layer "F.Cu") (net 3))
 (segment (start 53.80775 49.169) (end 53.80775 55.67775) (width 0.2) (layer "F.Cu") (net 3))
 (segment (start 121.24056 26.23825) (end 122.0465 27.04419) (width 0.2) (layer "F.Cu") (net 3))
 (segment (start 137.54425 47.309258) (end 130.763258 54.09025) (width 0.2) (layer "F.Cu") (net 3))
 (segment (start 136.06506 28.36275) (end 137.54425 29.84194) (width 0.2) (layer "F.Cu") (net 3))
 (segment (start 133.2636 27.05275) (end 133.2636 27.09565) (width 0.2) (layer "F.Cu") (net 3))
 (segment (start 54.6015 56.4715) (end 54.73 56.6) (width 0.2) (layer "F.Cu") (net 3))
 (segment (start 120.35994 26.23825) (end 121.24056 26.23825) (width 0.2) (layer "F.Cu") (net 3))
 (segment (start 133.2636 27.05275) (end 134.5736 28.36275) (width 0.2) (layer "F.Cu") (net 3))
 (segment (start 110.95775 55.80625) (end 111.7515 56.6) (width 0.2) (layer "F.Cu") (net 3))
 (segment (start 72.85775 49.169) (end 72.85775 55.80625) (width 0.2) (layer "F.Cu") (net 3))
 (segment (start 110.95775 49.169) (end 110.11622 49.169) (width 0.2) (layer "F.Cu") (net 3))
 (segment (start 110.95775 30.119) (end 113.18025 27.8965) (width 0.2) (layer "F.Cu") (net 3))
 (segment (start 92.7015 56.6) (end 111.7515 56.6) (width 0.2) (layer "F.Cu") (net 3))
 (segment (start 72.85775 30.119) (end 75.08025 27.8965) (width 0.2) (layer "F.Cu") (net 3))
 (segment (start 110.95775 49.169) (end 110.95775 55.80625) (width 0.2) (layer "F.Cu") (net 3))
 (segment (start 113.18025 27.8965) (end 115.125 29.84125) (width 0.2) (layer "F.Cu") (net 3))
 (segment (start 91.90775 30.119) (end 94.13025 27.8965) (width 0.2) (layer "F.Cu") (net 3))
 (segment (start 53.80775 55.67775) (end 54.6015 56.4715) (width 0.2) (layer "F.Cu") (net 3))
 (segment (start 134.5736 28.36275) (end 136.06506 28.36275) (width 0.2) (layer "F.Cu") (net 3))
 (segment (start 72.85775 49.169) (end 72.01622 49.169) (width 0.2) (layer "F.Cu") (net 3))
 (segment (start 122.0465 27.05275) (end 133.2636 27.05275) (width 0.2) (layer "F.Cu") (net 3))
 (segment (start 53.80775 30.119) (end 56.03025 27.8965) (width 0.2) (layer "F.Cu") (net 3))
 (segment (start 91.90775 49.169) (end 91.122934 49.169) (width 0.2) (layer "F.Cu") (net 3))
 (segment (start 75.08025 27.8965) (end 94.13025 27.8965) (width 0.2) (layer "F.Cu") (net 3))
 (segment (start 91.90775 49.169) (end 91.90775 55.80625) (width 0.2) (layer "F.Cu") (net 3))
 (segment (start 137.54425 29.84194) (end 137.54425 47.309258) (width 0.2) (layer "F.Cu") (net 3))
 (segment (start 122.0465 27.04419) (end 122.0465 27.05275) (width 0.2) (layer "F.Cu") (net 3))
 (segment (start 120.80025 29.84125) (end 119.73725 28.77825) (width 0.2) (layer "F.Cu") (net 3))
 (segment (start 94.13025 27.8965) (end 113.18025 27.8965) (width 0.2) (layer "F.Cu") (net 3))
 (segment (start 73.6515 56.6) (end 92.7015 56.6) (width 0.2) (layer "F.Cu") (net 3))
 (segment (start 126.2 29.4775) (end 123.5325 29.4775) (width 0.2) (layer "B.Cu") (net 3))
 (segment (start 125.14 34.24) (end 124.12 33.22) (width 0.2) (layer "B.Cu") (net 3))
 (segment (start 125.0275 39.0025) (end 125.01 39.02) (width 0.2) (layer "B.Cu") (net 3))
 (segment (start 126.2 34.24) (end 125.14 34.24) (width 0.2) (layer "B.Cu") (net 3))
 (segment (start 124.12 30.79) (end 123.17 29.84) (width 0.2) (layer "B.Cu") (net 3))
 (segment (start 124.12 38.13) (end 124.12 33.22) (width 0.2) (layer "B.Cu") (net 3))
 (segment (start 123.16875 29.84125) (end 120.80025 29.84125) (width 0.2) (layer "B.Cu") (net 3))
 (segment (start 125.01 39.02) (end 124.12 38.13) (width 0.2) (layer "B.Cu") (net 3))
 (segment (start 124.12 33.22) (end 124.12 30.79) (width 0.2) (layer "B.Cu") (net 3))
 (segment (start 123.5325 29.4775) (end 123.17 29.84) (width 0.2) (layer "B.Cu") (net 3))
 (segment (start 123.17 29.84) (end 123.16875 29.84125) (width 0.2) (layer "B.Cu") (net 3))
 (segment (start 126.2 39.0025) (end 125.0275 39.0025) (width 0.2) (layer "B.Cu") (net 3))
 (segment (start 136.04025 32.38125) (end 136.03875 32.38275) (width 0.2) (layer "F.Cu") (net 16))
 (segment (start 132.29 32.51) (end 132.41875 32.38125) (width 0.2) (layer "F.Cu") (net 16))
 (segment (start 132.41875 32.38125) (end 136.04025 32.38125) (width 0.2) (layer "F.Cu") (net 16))
 (via (at 132.29 32.51) (size 0.6) (drill 0.3) (layers "F.Cu" "B.Cu") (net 16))
 (segment (start 126.2 30.9775) (end 126.2 31.7) (width 0.2) (layer "B.Cu") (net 16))
 (segment (start 126.97 32.51) (end 127.001 32.479) (width 0.2) (layer "B.Cu") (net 16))
 (segment (start 126.2 31.7) (end 126.97 32.47) (width 0.2) (layer "B.Cu") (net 16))
 (segment (start 127.001 32.479) (end 132.259 32.479) (width 0.2) (layer "B.Cu") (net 16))
 (segment (start 126.97 32.47) (end 126.97 32.51) (width 0.2) (layer "B.Cu") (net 16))
 (segment (start 132.259 32.479) (end 132.29 32.51) (width 0.2) (layer "B.Cu") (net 16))
 (segment (start 132.2 35.74) (end 133.14 34.8) (width 0.2) (layer "B.Cu") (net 11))
 (segment (start 133.14 30.11) (end 133.14 28.74) (width 0.2) (layer "B.Cu") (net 11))
 (segment (start 133.14 39.5625) (end 133.14 34.8) (width 0.2) (layer "B.Cu") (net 11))
 (segment (start 133.14 28.74) (end 131.70125 27.30125) (width 0.2) (layer "B.Cu") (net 11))
 (segment (start 131.4 35.74) (end 132.2 35.74) (width 0.2) (layer "B.Cu") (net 11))
 (segment (start 131.4 40.5025) (end 132.2 40.5025) (width 0.2) (layer "B.Cu") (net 11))
 (segment (start 132.2 40.5025) (end 133.14 39.5625) (width 0.2) (layer "B.Cu") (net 11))
 (segment (start 131.4 30.9775) (end 132.2725 30.9775) (width 0.2) (layer "B.Cu") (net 11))
 (segment (start 131.70125 27.30125) (end 120.80025 27.30125) (width 0.2) (layer "B.Cu") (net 11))
 (segment (start 132.2725 30.9775) (end 133.14 30.11) (width 0.2) (layer "B.Cu") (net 11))
 (segment (start 133.14 34.8) (end 133.14 30.11) (width 0.2) (layer "B.Cu") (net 11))
 (segment (start 125.03 40.52) (end 125.03 38.48) (width 0.2) (layer "F.Cu") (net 13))
 (segment (start 131.45 33.09) (end 131.44 33.08) (width 0.2) (layer "F.Cu") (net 13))
 (segment (start 130.31 37.36) (end 130.58 37.36) (width 0.2) (layer "F.Cu") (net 13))
 (segment (start 125.03 38.48) (end 125.09 38.42) (width 0.2) (layer "F.Cu") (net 13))
 (segment (start 125.09 38.42) (end 126.15 37.36) (width 0.2) (layer "F.Cu") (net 13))
 (segment (start 126.15 37.36) (end 130.31 37.36) (width 0.2) (layer "F.Cu") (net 13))
 (segment (start 130.58 37.36) (end 131.45 36.49) (width 0.2) (layer "F.Cu") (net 13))
 (segment (start 131.45 36.49) (end 131.45 33.09) (width 0.2) (layer "F.Cu") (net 13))
 (via (at 131.44 33.08) (size 0.6) (drill 0.3) (layers "F.Cu" "B.Cu") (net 13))
 (via (at 125.03 40.52) (size 0.6) (drill 0.3) (layers "F.Cu" "B.Cu") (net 13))
 (segment (start 131.44 34.2) (end 131.4 34.24) (width 0.2) (layer "B.Cu") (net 13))
 (segment (start 125.0475 40.5025) (end 125.03 40.52) (width 0.2) (layer "B.Cu") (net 13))
 (segment (start 126.2 40.5025) (end 125.0475 40.5025) (width 0.2) (layer "B.Cu") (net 13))
 (segment (start 131.44 33.08) (end 131.44 34.2) (width 0.2) (layer "B.Cu") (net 13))
 (segment (start 108.96925 47.3475) (end 124.0005 47.3475) (width 0.2) (layer "F.Cu") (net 10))
 (segment (start 130.69879 46.9465) (end 135.10404 42.54125) (width 0.2) (layer "F.Cu") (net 10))
 (segment (start 104.60775 51.709) (end 108.96925 47.3475) (width 0.2) (layer "F.Cu") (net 10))
 (segment (start 124.0005 47.3475) (end 124.4015 46.9465) (width 0.2) (layer "F.Cu") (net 10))
 (segment (start 124.4015 46.9465) (end 130.69879 46.9465) (width 0.2) (layer "F.Cu") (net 10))
 (segment (start 135.10404 42.54125) (end 136.04025 42.54125) (width 0.2) (layer "F.Cu") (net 10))
 (segment (start 129.655142 55.761608) (end 128.8265 56.59025) (width 0.2) (layer "F.Cu") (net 2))
 (segment (start 129.659 55.761608) (end 129.655142 55.761608) (width 0.2) (layer "F.Cu") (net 2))
 (segment (start 137.94525 47.48275) (end 137.94525 29.20625) (width 0.2) (layer "F.Cu") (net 2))
 (segment (start 121.17025 56.59025) (end 128.8265 56.59025) (width 0.2) (layer "F.Cu") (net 2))
 (segment (start 137.94525 29.20625) (end 136.04025 27.30125) (width 0.2) (layer "F.Cu") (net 2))
 (segment (start 129.659 55.761608) (end 137.937858 47.48275) (width 0.2) (layer "F.Cu") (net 2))
 (segment (start 137.937858 47.48275) (end 137.94525 47.48275) (width 0.2) (layer "F.Cu") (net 2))
 (segment (start 137.10325 47.183158) (end 132.696158 51.59025) (width 0.2) (layer "F.Cu") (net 1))
 (segment (start 136.04025 29.84125) (end 137.10325 30.90425) (width 0.2) (layer "F.Cu") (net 1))
 (segment (start 136.04025 30.31084) (end 136.04025 29.84125) (width 0.2) (layer "F.Cu") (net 1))
 (segment (start 132.696158 51.59025) (end 121.17025 51.59025) (width 0.2) (layer "F.Cu") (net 1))
 (segment (start 137.10325 30.90425) (end 137.10325 47.183158) (width 0.2) (layer "F.Cu") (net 1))
 (segment (start 118.6117 40.3527) (end 118.6117 40.0863) (width 0.2) (layer "F.Cu") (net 9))
 (segment (start 118.6117 40.0863) (end 117.2784 38.753) (width 0.2) (layer "F.Cu") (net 9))
 (segment (start 51.1705 38.753) (end 47.45775 35.04025) (width 0.2) (layer "F.Cu") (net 9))
 (segment (start 120.80025 42.54125) (end 118.6117 40.3527) (width 0.2) (layer "F.Cu") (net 9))
 (segment (start 117.2784 38.753) (end 51.1705 38.753) (width 0.2) (layer "F.Cu") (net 9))
 (segment (start 47.45775 35.04025) (end 47.45775 32.659) (width 0.2) (layer "F.Cu") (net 9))
 (segment (start 120.80025 40.00125) (end 119.09375 40.00125) (width 0.2) (layer "F.Cu") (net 7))
 (segment (start 66.50775 35.04025) (end 66.50775 32.659) (width 0.2) (layer "F.Cu") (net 7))
 (segment (start 69.8195 38.352) (end 66.50775 35.04025) (width 0.2) (layer "F.Cu") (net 7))
 (segment (start 119.09375 40.00125) (end 117.4445 38.352) (width 0.2) (layer "F.Cu") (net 7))
 (segment (start 117.4445 38.352) (end 69.8195 38.352) (width 0.2) (layer "F.Cu") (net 7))
 (segment (start 87.88128 37.951) (end 120.3105 37.951) (width 0.2) (layer "F.Cu") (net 18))
 (segment (start 85.55775 32.659) (end 85.55775 35.62747) (width 0.2) (layer "F.Cu") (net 18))
 (segment (start 120.3105 37.951) (end 120.80025 37.46125) (width 0.2) (layer "F.Cu") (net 18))
 (segment (start 85.55775 35.62747) (end 87.88128 37.951) (width 0.2) (layer "F.Cu") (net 18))
 (segment (start 118.1715 37.55) (end 120.80025 34.92125) (width 0.2) (layer "F.Cu") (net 17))
 (segment (start 104.60775 32.659) (end 104.60775 35.04025) (width 0.2) (layer "F.Cu") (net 17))
 (segment (start 104.60775 35.04025) (end 107.1175 37.55) (width 0.2) (layer "F.Cu") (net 17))
 (segment (start 107.1175 37.55) (end 118.1715 37.55) (width 0.2) (layer "F.Cu") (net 17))
 (segment (start 71.10415 46.5455) (end 70.70315 46.9465) (width 0.2) (layer "F.Cu") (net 8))
 (segment (start 134.544545 41.399445) (end 134.544545 36.416955) (width 0.2) (layer "F.Cu") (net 8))
 (segment (start 52.22025 46.9465) (end 47.45775 51.709) (width 0.2) (layer "F.Cu") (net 8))
 (segment (start 89.98805 46.1445) (end 89.58705 46.5455) (width 0.2) (layer "F.Cu") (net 8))
 (segment (start 70.70315 46.9465) (end 52.22025 46.9465) (width 0.2) (layer "F.Cu") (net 8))
 (segment (start 123.49165 46.1445) (end 123.89265 45.7435) (width 0.2) (layer "F.Cu") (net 8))
 (segment (start 91.1365 46.1445) (end 123.49165 46.1445) (width 0.2) (layer "F.Cu") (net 8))
 (segment (start 89.58705 46.5455) (end 71.10415 46.5455) (width 0.2) (layer "F.Cu") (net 8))
 (segment (start 134.544545 36.416955) (end 136.04025 34.92125) (width 0.2) (layer "F.Cu") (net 8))
 (segment (start 123.89265 45.7435) (end 130.20049 45.7435) (width 0.2) (layer "F.Cu") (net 8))
 (segment (start 91.1365 46.1445) (end 89.98805 46.1445) (width 0.2) (layer "F.Cu") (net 8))
 (segment (start 130.20049 45.7435) (end 134.544545 41.399445) (width 0.2) (layer "F.Cu") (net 8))
 (segment (start 130.36659 46.1445) (end 134.945545 41.565545) (width 0.2) (layer "F.Cu") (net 14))
 (segment (start 90.15415 46.5455) (end 123.65775 46.5455) (width 0.2) (layer "F.Cu") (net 14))
 (segment (start 123.65775 46.5455) (end 124.05875 46.1445) (width 0.2) (layer "F.Cu") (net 14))
 (segment (start 66.50775 51.709) (end 71.27025 46.9465) (width 0.2) (layer "F.Cu") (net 14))
 (segment (start 134.945545 41.565545) (end 134.945545 38.555955) (width 0.2) (layer "F.Cu") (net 14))
 (segment (start 134.945545 38.555955) (end 136.04025 37.46125) (width 0.2) (layer "F.Cu") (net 14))
 (segment (start 89.75315 46.9465) (end 90.15415 46.5455) (width 0.2) (layer "F.Cu") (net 14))
 (segment (start 124.05875 46.1445) (end 130.36659 46.1445) (width 0.2) (layer "F.Cu") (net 14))
 (segment (start 71.27025 46.9465) (end 89.75315 46.9465) (width 0.2) (layer "F.Cu") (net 14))
 (segment (start 130.53269 46.5455) (end 136.04025 41.03794) (width 0.2) (layer "F.Cu") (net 6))
 (segment (start 90.32025 46.9465) (end 123.82385 46.9465) (width 0.2) (layer "F.Cu") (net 6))
 (segment (start 85.55775 51.709) (end 90.32025 46.9465) (width 0.2) (layer "F.Cu") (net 6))
 (segment (start 124.22485 46.5455) (end 130.53269 46.5455) (width 0.2) (layer "F.Cu") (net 6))
 (segment (start 123.82385 46.9465) (end 124.22485 46.5455) (width 0.2) (layer "F.Cu") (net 6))
 (segment (start 136.04025 41.03794) (end 136.04025 40.00125) (width 0.2) (layer "F.Cu") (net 6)))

